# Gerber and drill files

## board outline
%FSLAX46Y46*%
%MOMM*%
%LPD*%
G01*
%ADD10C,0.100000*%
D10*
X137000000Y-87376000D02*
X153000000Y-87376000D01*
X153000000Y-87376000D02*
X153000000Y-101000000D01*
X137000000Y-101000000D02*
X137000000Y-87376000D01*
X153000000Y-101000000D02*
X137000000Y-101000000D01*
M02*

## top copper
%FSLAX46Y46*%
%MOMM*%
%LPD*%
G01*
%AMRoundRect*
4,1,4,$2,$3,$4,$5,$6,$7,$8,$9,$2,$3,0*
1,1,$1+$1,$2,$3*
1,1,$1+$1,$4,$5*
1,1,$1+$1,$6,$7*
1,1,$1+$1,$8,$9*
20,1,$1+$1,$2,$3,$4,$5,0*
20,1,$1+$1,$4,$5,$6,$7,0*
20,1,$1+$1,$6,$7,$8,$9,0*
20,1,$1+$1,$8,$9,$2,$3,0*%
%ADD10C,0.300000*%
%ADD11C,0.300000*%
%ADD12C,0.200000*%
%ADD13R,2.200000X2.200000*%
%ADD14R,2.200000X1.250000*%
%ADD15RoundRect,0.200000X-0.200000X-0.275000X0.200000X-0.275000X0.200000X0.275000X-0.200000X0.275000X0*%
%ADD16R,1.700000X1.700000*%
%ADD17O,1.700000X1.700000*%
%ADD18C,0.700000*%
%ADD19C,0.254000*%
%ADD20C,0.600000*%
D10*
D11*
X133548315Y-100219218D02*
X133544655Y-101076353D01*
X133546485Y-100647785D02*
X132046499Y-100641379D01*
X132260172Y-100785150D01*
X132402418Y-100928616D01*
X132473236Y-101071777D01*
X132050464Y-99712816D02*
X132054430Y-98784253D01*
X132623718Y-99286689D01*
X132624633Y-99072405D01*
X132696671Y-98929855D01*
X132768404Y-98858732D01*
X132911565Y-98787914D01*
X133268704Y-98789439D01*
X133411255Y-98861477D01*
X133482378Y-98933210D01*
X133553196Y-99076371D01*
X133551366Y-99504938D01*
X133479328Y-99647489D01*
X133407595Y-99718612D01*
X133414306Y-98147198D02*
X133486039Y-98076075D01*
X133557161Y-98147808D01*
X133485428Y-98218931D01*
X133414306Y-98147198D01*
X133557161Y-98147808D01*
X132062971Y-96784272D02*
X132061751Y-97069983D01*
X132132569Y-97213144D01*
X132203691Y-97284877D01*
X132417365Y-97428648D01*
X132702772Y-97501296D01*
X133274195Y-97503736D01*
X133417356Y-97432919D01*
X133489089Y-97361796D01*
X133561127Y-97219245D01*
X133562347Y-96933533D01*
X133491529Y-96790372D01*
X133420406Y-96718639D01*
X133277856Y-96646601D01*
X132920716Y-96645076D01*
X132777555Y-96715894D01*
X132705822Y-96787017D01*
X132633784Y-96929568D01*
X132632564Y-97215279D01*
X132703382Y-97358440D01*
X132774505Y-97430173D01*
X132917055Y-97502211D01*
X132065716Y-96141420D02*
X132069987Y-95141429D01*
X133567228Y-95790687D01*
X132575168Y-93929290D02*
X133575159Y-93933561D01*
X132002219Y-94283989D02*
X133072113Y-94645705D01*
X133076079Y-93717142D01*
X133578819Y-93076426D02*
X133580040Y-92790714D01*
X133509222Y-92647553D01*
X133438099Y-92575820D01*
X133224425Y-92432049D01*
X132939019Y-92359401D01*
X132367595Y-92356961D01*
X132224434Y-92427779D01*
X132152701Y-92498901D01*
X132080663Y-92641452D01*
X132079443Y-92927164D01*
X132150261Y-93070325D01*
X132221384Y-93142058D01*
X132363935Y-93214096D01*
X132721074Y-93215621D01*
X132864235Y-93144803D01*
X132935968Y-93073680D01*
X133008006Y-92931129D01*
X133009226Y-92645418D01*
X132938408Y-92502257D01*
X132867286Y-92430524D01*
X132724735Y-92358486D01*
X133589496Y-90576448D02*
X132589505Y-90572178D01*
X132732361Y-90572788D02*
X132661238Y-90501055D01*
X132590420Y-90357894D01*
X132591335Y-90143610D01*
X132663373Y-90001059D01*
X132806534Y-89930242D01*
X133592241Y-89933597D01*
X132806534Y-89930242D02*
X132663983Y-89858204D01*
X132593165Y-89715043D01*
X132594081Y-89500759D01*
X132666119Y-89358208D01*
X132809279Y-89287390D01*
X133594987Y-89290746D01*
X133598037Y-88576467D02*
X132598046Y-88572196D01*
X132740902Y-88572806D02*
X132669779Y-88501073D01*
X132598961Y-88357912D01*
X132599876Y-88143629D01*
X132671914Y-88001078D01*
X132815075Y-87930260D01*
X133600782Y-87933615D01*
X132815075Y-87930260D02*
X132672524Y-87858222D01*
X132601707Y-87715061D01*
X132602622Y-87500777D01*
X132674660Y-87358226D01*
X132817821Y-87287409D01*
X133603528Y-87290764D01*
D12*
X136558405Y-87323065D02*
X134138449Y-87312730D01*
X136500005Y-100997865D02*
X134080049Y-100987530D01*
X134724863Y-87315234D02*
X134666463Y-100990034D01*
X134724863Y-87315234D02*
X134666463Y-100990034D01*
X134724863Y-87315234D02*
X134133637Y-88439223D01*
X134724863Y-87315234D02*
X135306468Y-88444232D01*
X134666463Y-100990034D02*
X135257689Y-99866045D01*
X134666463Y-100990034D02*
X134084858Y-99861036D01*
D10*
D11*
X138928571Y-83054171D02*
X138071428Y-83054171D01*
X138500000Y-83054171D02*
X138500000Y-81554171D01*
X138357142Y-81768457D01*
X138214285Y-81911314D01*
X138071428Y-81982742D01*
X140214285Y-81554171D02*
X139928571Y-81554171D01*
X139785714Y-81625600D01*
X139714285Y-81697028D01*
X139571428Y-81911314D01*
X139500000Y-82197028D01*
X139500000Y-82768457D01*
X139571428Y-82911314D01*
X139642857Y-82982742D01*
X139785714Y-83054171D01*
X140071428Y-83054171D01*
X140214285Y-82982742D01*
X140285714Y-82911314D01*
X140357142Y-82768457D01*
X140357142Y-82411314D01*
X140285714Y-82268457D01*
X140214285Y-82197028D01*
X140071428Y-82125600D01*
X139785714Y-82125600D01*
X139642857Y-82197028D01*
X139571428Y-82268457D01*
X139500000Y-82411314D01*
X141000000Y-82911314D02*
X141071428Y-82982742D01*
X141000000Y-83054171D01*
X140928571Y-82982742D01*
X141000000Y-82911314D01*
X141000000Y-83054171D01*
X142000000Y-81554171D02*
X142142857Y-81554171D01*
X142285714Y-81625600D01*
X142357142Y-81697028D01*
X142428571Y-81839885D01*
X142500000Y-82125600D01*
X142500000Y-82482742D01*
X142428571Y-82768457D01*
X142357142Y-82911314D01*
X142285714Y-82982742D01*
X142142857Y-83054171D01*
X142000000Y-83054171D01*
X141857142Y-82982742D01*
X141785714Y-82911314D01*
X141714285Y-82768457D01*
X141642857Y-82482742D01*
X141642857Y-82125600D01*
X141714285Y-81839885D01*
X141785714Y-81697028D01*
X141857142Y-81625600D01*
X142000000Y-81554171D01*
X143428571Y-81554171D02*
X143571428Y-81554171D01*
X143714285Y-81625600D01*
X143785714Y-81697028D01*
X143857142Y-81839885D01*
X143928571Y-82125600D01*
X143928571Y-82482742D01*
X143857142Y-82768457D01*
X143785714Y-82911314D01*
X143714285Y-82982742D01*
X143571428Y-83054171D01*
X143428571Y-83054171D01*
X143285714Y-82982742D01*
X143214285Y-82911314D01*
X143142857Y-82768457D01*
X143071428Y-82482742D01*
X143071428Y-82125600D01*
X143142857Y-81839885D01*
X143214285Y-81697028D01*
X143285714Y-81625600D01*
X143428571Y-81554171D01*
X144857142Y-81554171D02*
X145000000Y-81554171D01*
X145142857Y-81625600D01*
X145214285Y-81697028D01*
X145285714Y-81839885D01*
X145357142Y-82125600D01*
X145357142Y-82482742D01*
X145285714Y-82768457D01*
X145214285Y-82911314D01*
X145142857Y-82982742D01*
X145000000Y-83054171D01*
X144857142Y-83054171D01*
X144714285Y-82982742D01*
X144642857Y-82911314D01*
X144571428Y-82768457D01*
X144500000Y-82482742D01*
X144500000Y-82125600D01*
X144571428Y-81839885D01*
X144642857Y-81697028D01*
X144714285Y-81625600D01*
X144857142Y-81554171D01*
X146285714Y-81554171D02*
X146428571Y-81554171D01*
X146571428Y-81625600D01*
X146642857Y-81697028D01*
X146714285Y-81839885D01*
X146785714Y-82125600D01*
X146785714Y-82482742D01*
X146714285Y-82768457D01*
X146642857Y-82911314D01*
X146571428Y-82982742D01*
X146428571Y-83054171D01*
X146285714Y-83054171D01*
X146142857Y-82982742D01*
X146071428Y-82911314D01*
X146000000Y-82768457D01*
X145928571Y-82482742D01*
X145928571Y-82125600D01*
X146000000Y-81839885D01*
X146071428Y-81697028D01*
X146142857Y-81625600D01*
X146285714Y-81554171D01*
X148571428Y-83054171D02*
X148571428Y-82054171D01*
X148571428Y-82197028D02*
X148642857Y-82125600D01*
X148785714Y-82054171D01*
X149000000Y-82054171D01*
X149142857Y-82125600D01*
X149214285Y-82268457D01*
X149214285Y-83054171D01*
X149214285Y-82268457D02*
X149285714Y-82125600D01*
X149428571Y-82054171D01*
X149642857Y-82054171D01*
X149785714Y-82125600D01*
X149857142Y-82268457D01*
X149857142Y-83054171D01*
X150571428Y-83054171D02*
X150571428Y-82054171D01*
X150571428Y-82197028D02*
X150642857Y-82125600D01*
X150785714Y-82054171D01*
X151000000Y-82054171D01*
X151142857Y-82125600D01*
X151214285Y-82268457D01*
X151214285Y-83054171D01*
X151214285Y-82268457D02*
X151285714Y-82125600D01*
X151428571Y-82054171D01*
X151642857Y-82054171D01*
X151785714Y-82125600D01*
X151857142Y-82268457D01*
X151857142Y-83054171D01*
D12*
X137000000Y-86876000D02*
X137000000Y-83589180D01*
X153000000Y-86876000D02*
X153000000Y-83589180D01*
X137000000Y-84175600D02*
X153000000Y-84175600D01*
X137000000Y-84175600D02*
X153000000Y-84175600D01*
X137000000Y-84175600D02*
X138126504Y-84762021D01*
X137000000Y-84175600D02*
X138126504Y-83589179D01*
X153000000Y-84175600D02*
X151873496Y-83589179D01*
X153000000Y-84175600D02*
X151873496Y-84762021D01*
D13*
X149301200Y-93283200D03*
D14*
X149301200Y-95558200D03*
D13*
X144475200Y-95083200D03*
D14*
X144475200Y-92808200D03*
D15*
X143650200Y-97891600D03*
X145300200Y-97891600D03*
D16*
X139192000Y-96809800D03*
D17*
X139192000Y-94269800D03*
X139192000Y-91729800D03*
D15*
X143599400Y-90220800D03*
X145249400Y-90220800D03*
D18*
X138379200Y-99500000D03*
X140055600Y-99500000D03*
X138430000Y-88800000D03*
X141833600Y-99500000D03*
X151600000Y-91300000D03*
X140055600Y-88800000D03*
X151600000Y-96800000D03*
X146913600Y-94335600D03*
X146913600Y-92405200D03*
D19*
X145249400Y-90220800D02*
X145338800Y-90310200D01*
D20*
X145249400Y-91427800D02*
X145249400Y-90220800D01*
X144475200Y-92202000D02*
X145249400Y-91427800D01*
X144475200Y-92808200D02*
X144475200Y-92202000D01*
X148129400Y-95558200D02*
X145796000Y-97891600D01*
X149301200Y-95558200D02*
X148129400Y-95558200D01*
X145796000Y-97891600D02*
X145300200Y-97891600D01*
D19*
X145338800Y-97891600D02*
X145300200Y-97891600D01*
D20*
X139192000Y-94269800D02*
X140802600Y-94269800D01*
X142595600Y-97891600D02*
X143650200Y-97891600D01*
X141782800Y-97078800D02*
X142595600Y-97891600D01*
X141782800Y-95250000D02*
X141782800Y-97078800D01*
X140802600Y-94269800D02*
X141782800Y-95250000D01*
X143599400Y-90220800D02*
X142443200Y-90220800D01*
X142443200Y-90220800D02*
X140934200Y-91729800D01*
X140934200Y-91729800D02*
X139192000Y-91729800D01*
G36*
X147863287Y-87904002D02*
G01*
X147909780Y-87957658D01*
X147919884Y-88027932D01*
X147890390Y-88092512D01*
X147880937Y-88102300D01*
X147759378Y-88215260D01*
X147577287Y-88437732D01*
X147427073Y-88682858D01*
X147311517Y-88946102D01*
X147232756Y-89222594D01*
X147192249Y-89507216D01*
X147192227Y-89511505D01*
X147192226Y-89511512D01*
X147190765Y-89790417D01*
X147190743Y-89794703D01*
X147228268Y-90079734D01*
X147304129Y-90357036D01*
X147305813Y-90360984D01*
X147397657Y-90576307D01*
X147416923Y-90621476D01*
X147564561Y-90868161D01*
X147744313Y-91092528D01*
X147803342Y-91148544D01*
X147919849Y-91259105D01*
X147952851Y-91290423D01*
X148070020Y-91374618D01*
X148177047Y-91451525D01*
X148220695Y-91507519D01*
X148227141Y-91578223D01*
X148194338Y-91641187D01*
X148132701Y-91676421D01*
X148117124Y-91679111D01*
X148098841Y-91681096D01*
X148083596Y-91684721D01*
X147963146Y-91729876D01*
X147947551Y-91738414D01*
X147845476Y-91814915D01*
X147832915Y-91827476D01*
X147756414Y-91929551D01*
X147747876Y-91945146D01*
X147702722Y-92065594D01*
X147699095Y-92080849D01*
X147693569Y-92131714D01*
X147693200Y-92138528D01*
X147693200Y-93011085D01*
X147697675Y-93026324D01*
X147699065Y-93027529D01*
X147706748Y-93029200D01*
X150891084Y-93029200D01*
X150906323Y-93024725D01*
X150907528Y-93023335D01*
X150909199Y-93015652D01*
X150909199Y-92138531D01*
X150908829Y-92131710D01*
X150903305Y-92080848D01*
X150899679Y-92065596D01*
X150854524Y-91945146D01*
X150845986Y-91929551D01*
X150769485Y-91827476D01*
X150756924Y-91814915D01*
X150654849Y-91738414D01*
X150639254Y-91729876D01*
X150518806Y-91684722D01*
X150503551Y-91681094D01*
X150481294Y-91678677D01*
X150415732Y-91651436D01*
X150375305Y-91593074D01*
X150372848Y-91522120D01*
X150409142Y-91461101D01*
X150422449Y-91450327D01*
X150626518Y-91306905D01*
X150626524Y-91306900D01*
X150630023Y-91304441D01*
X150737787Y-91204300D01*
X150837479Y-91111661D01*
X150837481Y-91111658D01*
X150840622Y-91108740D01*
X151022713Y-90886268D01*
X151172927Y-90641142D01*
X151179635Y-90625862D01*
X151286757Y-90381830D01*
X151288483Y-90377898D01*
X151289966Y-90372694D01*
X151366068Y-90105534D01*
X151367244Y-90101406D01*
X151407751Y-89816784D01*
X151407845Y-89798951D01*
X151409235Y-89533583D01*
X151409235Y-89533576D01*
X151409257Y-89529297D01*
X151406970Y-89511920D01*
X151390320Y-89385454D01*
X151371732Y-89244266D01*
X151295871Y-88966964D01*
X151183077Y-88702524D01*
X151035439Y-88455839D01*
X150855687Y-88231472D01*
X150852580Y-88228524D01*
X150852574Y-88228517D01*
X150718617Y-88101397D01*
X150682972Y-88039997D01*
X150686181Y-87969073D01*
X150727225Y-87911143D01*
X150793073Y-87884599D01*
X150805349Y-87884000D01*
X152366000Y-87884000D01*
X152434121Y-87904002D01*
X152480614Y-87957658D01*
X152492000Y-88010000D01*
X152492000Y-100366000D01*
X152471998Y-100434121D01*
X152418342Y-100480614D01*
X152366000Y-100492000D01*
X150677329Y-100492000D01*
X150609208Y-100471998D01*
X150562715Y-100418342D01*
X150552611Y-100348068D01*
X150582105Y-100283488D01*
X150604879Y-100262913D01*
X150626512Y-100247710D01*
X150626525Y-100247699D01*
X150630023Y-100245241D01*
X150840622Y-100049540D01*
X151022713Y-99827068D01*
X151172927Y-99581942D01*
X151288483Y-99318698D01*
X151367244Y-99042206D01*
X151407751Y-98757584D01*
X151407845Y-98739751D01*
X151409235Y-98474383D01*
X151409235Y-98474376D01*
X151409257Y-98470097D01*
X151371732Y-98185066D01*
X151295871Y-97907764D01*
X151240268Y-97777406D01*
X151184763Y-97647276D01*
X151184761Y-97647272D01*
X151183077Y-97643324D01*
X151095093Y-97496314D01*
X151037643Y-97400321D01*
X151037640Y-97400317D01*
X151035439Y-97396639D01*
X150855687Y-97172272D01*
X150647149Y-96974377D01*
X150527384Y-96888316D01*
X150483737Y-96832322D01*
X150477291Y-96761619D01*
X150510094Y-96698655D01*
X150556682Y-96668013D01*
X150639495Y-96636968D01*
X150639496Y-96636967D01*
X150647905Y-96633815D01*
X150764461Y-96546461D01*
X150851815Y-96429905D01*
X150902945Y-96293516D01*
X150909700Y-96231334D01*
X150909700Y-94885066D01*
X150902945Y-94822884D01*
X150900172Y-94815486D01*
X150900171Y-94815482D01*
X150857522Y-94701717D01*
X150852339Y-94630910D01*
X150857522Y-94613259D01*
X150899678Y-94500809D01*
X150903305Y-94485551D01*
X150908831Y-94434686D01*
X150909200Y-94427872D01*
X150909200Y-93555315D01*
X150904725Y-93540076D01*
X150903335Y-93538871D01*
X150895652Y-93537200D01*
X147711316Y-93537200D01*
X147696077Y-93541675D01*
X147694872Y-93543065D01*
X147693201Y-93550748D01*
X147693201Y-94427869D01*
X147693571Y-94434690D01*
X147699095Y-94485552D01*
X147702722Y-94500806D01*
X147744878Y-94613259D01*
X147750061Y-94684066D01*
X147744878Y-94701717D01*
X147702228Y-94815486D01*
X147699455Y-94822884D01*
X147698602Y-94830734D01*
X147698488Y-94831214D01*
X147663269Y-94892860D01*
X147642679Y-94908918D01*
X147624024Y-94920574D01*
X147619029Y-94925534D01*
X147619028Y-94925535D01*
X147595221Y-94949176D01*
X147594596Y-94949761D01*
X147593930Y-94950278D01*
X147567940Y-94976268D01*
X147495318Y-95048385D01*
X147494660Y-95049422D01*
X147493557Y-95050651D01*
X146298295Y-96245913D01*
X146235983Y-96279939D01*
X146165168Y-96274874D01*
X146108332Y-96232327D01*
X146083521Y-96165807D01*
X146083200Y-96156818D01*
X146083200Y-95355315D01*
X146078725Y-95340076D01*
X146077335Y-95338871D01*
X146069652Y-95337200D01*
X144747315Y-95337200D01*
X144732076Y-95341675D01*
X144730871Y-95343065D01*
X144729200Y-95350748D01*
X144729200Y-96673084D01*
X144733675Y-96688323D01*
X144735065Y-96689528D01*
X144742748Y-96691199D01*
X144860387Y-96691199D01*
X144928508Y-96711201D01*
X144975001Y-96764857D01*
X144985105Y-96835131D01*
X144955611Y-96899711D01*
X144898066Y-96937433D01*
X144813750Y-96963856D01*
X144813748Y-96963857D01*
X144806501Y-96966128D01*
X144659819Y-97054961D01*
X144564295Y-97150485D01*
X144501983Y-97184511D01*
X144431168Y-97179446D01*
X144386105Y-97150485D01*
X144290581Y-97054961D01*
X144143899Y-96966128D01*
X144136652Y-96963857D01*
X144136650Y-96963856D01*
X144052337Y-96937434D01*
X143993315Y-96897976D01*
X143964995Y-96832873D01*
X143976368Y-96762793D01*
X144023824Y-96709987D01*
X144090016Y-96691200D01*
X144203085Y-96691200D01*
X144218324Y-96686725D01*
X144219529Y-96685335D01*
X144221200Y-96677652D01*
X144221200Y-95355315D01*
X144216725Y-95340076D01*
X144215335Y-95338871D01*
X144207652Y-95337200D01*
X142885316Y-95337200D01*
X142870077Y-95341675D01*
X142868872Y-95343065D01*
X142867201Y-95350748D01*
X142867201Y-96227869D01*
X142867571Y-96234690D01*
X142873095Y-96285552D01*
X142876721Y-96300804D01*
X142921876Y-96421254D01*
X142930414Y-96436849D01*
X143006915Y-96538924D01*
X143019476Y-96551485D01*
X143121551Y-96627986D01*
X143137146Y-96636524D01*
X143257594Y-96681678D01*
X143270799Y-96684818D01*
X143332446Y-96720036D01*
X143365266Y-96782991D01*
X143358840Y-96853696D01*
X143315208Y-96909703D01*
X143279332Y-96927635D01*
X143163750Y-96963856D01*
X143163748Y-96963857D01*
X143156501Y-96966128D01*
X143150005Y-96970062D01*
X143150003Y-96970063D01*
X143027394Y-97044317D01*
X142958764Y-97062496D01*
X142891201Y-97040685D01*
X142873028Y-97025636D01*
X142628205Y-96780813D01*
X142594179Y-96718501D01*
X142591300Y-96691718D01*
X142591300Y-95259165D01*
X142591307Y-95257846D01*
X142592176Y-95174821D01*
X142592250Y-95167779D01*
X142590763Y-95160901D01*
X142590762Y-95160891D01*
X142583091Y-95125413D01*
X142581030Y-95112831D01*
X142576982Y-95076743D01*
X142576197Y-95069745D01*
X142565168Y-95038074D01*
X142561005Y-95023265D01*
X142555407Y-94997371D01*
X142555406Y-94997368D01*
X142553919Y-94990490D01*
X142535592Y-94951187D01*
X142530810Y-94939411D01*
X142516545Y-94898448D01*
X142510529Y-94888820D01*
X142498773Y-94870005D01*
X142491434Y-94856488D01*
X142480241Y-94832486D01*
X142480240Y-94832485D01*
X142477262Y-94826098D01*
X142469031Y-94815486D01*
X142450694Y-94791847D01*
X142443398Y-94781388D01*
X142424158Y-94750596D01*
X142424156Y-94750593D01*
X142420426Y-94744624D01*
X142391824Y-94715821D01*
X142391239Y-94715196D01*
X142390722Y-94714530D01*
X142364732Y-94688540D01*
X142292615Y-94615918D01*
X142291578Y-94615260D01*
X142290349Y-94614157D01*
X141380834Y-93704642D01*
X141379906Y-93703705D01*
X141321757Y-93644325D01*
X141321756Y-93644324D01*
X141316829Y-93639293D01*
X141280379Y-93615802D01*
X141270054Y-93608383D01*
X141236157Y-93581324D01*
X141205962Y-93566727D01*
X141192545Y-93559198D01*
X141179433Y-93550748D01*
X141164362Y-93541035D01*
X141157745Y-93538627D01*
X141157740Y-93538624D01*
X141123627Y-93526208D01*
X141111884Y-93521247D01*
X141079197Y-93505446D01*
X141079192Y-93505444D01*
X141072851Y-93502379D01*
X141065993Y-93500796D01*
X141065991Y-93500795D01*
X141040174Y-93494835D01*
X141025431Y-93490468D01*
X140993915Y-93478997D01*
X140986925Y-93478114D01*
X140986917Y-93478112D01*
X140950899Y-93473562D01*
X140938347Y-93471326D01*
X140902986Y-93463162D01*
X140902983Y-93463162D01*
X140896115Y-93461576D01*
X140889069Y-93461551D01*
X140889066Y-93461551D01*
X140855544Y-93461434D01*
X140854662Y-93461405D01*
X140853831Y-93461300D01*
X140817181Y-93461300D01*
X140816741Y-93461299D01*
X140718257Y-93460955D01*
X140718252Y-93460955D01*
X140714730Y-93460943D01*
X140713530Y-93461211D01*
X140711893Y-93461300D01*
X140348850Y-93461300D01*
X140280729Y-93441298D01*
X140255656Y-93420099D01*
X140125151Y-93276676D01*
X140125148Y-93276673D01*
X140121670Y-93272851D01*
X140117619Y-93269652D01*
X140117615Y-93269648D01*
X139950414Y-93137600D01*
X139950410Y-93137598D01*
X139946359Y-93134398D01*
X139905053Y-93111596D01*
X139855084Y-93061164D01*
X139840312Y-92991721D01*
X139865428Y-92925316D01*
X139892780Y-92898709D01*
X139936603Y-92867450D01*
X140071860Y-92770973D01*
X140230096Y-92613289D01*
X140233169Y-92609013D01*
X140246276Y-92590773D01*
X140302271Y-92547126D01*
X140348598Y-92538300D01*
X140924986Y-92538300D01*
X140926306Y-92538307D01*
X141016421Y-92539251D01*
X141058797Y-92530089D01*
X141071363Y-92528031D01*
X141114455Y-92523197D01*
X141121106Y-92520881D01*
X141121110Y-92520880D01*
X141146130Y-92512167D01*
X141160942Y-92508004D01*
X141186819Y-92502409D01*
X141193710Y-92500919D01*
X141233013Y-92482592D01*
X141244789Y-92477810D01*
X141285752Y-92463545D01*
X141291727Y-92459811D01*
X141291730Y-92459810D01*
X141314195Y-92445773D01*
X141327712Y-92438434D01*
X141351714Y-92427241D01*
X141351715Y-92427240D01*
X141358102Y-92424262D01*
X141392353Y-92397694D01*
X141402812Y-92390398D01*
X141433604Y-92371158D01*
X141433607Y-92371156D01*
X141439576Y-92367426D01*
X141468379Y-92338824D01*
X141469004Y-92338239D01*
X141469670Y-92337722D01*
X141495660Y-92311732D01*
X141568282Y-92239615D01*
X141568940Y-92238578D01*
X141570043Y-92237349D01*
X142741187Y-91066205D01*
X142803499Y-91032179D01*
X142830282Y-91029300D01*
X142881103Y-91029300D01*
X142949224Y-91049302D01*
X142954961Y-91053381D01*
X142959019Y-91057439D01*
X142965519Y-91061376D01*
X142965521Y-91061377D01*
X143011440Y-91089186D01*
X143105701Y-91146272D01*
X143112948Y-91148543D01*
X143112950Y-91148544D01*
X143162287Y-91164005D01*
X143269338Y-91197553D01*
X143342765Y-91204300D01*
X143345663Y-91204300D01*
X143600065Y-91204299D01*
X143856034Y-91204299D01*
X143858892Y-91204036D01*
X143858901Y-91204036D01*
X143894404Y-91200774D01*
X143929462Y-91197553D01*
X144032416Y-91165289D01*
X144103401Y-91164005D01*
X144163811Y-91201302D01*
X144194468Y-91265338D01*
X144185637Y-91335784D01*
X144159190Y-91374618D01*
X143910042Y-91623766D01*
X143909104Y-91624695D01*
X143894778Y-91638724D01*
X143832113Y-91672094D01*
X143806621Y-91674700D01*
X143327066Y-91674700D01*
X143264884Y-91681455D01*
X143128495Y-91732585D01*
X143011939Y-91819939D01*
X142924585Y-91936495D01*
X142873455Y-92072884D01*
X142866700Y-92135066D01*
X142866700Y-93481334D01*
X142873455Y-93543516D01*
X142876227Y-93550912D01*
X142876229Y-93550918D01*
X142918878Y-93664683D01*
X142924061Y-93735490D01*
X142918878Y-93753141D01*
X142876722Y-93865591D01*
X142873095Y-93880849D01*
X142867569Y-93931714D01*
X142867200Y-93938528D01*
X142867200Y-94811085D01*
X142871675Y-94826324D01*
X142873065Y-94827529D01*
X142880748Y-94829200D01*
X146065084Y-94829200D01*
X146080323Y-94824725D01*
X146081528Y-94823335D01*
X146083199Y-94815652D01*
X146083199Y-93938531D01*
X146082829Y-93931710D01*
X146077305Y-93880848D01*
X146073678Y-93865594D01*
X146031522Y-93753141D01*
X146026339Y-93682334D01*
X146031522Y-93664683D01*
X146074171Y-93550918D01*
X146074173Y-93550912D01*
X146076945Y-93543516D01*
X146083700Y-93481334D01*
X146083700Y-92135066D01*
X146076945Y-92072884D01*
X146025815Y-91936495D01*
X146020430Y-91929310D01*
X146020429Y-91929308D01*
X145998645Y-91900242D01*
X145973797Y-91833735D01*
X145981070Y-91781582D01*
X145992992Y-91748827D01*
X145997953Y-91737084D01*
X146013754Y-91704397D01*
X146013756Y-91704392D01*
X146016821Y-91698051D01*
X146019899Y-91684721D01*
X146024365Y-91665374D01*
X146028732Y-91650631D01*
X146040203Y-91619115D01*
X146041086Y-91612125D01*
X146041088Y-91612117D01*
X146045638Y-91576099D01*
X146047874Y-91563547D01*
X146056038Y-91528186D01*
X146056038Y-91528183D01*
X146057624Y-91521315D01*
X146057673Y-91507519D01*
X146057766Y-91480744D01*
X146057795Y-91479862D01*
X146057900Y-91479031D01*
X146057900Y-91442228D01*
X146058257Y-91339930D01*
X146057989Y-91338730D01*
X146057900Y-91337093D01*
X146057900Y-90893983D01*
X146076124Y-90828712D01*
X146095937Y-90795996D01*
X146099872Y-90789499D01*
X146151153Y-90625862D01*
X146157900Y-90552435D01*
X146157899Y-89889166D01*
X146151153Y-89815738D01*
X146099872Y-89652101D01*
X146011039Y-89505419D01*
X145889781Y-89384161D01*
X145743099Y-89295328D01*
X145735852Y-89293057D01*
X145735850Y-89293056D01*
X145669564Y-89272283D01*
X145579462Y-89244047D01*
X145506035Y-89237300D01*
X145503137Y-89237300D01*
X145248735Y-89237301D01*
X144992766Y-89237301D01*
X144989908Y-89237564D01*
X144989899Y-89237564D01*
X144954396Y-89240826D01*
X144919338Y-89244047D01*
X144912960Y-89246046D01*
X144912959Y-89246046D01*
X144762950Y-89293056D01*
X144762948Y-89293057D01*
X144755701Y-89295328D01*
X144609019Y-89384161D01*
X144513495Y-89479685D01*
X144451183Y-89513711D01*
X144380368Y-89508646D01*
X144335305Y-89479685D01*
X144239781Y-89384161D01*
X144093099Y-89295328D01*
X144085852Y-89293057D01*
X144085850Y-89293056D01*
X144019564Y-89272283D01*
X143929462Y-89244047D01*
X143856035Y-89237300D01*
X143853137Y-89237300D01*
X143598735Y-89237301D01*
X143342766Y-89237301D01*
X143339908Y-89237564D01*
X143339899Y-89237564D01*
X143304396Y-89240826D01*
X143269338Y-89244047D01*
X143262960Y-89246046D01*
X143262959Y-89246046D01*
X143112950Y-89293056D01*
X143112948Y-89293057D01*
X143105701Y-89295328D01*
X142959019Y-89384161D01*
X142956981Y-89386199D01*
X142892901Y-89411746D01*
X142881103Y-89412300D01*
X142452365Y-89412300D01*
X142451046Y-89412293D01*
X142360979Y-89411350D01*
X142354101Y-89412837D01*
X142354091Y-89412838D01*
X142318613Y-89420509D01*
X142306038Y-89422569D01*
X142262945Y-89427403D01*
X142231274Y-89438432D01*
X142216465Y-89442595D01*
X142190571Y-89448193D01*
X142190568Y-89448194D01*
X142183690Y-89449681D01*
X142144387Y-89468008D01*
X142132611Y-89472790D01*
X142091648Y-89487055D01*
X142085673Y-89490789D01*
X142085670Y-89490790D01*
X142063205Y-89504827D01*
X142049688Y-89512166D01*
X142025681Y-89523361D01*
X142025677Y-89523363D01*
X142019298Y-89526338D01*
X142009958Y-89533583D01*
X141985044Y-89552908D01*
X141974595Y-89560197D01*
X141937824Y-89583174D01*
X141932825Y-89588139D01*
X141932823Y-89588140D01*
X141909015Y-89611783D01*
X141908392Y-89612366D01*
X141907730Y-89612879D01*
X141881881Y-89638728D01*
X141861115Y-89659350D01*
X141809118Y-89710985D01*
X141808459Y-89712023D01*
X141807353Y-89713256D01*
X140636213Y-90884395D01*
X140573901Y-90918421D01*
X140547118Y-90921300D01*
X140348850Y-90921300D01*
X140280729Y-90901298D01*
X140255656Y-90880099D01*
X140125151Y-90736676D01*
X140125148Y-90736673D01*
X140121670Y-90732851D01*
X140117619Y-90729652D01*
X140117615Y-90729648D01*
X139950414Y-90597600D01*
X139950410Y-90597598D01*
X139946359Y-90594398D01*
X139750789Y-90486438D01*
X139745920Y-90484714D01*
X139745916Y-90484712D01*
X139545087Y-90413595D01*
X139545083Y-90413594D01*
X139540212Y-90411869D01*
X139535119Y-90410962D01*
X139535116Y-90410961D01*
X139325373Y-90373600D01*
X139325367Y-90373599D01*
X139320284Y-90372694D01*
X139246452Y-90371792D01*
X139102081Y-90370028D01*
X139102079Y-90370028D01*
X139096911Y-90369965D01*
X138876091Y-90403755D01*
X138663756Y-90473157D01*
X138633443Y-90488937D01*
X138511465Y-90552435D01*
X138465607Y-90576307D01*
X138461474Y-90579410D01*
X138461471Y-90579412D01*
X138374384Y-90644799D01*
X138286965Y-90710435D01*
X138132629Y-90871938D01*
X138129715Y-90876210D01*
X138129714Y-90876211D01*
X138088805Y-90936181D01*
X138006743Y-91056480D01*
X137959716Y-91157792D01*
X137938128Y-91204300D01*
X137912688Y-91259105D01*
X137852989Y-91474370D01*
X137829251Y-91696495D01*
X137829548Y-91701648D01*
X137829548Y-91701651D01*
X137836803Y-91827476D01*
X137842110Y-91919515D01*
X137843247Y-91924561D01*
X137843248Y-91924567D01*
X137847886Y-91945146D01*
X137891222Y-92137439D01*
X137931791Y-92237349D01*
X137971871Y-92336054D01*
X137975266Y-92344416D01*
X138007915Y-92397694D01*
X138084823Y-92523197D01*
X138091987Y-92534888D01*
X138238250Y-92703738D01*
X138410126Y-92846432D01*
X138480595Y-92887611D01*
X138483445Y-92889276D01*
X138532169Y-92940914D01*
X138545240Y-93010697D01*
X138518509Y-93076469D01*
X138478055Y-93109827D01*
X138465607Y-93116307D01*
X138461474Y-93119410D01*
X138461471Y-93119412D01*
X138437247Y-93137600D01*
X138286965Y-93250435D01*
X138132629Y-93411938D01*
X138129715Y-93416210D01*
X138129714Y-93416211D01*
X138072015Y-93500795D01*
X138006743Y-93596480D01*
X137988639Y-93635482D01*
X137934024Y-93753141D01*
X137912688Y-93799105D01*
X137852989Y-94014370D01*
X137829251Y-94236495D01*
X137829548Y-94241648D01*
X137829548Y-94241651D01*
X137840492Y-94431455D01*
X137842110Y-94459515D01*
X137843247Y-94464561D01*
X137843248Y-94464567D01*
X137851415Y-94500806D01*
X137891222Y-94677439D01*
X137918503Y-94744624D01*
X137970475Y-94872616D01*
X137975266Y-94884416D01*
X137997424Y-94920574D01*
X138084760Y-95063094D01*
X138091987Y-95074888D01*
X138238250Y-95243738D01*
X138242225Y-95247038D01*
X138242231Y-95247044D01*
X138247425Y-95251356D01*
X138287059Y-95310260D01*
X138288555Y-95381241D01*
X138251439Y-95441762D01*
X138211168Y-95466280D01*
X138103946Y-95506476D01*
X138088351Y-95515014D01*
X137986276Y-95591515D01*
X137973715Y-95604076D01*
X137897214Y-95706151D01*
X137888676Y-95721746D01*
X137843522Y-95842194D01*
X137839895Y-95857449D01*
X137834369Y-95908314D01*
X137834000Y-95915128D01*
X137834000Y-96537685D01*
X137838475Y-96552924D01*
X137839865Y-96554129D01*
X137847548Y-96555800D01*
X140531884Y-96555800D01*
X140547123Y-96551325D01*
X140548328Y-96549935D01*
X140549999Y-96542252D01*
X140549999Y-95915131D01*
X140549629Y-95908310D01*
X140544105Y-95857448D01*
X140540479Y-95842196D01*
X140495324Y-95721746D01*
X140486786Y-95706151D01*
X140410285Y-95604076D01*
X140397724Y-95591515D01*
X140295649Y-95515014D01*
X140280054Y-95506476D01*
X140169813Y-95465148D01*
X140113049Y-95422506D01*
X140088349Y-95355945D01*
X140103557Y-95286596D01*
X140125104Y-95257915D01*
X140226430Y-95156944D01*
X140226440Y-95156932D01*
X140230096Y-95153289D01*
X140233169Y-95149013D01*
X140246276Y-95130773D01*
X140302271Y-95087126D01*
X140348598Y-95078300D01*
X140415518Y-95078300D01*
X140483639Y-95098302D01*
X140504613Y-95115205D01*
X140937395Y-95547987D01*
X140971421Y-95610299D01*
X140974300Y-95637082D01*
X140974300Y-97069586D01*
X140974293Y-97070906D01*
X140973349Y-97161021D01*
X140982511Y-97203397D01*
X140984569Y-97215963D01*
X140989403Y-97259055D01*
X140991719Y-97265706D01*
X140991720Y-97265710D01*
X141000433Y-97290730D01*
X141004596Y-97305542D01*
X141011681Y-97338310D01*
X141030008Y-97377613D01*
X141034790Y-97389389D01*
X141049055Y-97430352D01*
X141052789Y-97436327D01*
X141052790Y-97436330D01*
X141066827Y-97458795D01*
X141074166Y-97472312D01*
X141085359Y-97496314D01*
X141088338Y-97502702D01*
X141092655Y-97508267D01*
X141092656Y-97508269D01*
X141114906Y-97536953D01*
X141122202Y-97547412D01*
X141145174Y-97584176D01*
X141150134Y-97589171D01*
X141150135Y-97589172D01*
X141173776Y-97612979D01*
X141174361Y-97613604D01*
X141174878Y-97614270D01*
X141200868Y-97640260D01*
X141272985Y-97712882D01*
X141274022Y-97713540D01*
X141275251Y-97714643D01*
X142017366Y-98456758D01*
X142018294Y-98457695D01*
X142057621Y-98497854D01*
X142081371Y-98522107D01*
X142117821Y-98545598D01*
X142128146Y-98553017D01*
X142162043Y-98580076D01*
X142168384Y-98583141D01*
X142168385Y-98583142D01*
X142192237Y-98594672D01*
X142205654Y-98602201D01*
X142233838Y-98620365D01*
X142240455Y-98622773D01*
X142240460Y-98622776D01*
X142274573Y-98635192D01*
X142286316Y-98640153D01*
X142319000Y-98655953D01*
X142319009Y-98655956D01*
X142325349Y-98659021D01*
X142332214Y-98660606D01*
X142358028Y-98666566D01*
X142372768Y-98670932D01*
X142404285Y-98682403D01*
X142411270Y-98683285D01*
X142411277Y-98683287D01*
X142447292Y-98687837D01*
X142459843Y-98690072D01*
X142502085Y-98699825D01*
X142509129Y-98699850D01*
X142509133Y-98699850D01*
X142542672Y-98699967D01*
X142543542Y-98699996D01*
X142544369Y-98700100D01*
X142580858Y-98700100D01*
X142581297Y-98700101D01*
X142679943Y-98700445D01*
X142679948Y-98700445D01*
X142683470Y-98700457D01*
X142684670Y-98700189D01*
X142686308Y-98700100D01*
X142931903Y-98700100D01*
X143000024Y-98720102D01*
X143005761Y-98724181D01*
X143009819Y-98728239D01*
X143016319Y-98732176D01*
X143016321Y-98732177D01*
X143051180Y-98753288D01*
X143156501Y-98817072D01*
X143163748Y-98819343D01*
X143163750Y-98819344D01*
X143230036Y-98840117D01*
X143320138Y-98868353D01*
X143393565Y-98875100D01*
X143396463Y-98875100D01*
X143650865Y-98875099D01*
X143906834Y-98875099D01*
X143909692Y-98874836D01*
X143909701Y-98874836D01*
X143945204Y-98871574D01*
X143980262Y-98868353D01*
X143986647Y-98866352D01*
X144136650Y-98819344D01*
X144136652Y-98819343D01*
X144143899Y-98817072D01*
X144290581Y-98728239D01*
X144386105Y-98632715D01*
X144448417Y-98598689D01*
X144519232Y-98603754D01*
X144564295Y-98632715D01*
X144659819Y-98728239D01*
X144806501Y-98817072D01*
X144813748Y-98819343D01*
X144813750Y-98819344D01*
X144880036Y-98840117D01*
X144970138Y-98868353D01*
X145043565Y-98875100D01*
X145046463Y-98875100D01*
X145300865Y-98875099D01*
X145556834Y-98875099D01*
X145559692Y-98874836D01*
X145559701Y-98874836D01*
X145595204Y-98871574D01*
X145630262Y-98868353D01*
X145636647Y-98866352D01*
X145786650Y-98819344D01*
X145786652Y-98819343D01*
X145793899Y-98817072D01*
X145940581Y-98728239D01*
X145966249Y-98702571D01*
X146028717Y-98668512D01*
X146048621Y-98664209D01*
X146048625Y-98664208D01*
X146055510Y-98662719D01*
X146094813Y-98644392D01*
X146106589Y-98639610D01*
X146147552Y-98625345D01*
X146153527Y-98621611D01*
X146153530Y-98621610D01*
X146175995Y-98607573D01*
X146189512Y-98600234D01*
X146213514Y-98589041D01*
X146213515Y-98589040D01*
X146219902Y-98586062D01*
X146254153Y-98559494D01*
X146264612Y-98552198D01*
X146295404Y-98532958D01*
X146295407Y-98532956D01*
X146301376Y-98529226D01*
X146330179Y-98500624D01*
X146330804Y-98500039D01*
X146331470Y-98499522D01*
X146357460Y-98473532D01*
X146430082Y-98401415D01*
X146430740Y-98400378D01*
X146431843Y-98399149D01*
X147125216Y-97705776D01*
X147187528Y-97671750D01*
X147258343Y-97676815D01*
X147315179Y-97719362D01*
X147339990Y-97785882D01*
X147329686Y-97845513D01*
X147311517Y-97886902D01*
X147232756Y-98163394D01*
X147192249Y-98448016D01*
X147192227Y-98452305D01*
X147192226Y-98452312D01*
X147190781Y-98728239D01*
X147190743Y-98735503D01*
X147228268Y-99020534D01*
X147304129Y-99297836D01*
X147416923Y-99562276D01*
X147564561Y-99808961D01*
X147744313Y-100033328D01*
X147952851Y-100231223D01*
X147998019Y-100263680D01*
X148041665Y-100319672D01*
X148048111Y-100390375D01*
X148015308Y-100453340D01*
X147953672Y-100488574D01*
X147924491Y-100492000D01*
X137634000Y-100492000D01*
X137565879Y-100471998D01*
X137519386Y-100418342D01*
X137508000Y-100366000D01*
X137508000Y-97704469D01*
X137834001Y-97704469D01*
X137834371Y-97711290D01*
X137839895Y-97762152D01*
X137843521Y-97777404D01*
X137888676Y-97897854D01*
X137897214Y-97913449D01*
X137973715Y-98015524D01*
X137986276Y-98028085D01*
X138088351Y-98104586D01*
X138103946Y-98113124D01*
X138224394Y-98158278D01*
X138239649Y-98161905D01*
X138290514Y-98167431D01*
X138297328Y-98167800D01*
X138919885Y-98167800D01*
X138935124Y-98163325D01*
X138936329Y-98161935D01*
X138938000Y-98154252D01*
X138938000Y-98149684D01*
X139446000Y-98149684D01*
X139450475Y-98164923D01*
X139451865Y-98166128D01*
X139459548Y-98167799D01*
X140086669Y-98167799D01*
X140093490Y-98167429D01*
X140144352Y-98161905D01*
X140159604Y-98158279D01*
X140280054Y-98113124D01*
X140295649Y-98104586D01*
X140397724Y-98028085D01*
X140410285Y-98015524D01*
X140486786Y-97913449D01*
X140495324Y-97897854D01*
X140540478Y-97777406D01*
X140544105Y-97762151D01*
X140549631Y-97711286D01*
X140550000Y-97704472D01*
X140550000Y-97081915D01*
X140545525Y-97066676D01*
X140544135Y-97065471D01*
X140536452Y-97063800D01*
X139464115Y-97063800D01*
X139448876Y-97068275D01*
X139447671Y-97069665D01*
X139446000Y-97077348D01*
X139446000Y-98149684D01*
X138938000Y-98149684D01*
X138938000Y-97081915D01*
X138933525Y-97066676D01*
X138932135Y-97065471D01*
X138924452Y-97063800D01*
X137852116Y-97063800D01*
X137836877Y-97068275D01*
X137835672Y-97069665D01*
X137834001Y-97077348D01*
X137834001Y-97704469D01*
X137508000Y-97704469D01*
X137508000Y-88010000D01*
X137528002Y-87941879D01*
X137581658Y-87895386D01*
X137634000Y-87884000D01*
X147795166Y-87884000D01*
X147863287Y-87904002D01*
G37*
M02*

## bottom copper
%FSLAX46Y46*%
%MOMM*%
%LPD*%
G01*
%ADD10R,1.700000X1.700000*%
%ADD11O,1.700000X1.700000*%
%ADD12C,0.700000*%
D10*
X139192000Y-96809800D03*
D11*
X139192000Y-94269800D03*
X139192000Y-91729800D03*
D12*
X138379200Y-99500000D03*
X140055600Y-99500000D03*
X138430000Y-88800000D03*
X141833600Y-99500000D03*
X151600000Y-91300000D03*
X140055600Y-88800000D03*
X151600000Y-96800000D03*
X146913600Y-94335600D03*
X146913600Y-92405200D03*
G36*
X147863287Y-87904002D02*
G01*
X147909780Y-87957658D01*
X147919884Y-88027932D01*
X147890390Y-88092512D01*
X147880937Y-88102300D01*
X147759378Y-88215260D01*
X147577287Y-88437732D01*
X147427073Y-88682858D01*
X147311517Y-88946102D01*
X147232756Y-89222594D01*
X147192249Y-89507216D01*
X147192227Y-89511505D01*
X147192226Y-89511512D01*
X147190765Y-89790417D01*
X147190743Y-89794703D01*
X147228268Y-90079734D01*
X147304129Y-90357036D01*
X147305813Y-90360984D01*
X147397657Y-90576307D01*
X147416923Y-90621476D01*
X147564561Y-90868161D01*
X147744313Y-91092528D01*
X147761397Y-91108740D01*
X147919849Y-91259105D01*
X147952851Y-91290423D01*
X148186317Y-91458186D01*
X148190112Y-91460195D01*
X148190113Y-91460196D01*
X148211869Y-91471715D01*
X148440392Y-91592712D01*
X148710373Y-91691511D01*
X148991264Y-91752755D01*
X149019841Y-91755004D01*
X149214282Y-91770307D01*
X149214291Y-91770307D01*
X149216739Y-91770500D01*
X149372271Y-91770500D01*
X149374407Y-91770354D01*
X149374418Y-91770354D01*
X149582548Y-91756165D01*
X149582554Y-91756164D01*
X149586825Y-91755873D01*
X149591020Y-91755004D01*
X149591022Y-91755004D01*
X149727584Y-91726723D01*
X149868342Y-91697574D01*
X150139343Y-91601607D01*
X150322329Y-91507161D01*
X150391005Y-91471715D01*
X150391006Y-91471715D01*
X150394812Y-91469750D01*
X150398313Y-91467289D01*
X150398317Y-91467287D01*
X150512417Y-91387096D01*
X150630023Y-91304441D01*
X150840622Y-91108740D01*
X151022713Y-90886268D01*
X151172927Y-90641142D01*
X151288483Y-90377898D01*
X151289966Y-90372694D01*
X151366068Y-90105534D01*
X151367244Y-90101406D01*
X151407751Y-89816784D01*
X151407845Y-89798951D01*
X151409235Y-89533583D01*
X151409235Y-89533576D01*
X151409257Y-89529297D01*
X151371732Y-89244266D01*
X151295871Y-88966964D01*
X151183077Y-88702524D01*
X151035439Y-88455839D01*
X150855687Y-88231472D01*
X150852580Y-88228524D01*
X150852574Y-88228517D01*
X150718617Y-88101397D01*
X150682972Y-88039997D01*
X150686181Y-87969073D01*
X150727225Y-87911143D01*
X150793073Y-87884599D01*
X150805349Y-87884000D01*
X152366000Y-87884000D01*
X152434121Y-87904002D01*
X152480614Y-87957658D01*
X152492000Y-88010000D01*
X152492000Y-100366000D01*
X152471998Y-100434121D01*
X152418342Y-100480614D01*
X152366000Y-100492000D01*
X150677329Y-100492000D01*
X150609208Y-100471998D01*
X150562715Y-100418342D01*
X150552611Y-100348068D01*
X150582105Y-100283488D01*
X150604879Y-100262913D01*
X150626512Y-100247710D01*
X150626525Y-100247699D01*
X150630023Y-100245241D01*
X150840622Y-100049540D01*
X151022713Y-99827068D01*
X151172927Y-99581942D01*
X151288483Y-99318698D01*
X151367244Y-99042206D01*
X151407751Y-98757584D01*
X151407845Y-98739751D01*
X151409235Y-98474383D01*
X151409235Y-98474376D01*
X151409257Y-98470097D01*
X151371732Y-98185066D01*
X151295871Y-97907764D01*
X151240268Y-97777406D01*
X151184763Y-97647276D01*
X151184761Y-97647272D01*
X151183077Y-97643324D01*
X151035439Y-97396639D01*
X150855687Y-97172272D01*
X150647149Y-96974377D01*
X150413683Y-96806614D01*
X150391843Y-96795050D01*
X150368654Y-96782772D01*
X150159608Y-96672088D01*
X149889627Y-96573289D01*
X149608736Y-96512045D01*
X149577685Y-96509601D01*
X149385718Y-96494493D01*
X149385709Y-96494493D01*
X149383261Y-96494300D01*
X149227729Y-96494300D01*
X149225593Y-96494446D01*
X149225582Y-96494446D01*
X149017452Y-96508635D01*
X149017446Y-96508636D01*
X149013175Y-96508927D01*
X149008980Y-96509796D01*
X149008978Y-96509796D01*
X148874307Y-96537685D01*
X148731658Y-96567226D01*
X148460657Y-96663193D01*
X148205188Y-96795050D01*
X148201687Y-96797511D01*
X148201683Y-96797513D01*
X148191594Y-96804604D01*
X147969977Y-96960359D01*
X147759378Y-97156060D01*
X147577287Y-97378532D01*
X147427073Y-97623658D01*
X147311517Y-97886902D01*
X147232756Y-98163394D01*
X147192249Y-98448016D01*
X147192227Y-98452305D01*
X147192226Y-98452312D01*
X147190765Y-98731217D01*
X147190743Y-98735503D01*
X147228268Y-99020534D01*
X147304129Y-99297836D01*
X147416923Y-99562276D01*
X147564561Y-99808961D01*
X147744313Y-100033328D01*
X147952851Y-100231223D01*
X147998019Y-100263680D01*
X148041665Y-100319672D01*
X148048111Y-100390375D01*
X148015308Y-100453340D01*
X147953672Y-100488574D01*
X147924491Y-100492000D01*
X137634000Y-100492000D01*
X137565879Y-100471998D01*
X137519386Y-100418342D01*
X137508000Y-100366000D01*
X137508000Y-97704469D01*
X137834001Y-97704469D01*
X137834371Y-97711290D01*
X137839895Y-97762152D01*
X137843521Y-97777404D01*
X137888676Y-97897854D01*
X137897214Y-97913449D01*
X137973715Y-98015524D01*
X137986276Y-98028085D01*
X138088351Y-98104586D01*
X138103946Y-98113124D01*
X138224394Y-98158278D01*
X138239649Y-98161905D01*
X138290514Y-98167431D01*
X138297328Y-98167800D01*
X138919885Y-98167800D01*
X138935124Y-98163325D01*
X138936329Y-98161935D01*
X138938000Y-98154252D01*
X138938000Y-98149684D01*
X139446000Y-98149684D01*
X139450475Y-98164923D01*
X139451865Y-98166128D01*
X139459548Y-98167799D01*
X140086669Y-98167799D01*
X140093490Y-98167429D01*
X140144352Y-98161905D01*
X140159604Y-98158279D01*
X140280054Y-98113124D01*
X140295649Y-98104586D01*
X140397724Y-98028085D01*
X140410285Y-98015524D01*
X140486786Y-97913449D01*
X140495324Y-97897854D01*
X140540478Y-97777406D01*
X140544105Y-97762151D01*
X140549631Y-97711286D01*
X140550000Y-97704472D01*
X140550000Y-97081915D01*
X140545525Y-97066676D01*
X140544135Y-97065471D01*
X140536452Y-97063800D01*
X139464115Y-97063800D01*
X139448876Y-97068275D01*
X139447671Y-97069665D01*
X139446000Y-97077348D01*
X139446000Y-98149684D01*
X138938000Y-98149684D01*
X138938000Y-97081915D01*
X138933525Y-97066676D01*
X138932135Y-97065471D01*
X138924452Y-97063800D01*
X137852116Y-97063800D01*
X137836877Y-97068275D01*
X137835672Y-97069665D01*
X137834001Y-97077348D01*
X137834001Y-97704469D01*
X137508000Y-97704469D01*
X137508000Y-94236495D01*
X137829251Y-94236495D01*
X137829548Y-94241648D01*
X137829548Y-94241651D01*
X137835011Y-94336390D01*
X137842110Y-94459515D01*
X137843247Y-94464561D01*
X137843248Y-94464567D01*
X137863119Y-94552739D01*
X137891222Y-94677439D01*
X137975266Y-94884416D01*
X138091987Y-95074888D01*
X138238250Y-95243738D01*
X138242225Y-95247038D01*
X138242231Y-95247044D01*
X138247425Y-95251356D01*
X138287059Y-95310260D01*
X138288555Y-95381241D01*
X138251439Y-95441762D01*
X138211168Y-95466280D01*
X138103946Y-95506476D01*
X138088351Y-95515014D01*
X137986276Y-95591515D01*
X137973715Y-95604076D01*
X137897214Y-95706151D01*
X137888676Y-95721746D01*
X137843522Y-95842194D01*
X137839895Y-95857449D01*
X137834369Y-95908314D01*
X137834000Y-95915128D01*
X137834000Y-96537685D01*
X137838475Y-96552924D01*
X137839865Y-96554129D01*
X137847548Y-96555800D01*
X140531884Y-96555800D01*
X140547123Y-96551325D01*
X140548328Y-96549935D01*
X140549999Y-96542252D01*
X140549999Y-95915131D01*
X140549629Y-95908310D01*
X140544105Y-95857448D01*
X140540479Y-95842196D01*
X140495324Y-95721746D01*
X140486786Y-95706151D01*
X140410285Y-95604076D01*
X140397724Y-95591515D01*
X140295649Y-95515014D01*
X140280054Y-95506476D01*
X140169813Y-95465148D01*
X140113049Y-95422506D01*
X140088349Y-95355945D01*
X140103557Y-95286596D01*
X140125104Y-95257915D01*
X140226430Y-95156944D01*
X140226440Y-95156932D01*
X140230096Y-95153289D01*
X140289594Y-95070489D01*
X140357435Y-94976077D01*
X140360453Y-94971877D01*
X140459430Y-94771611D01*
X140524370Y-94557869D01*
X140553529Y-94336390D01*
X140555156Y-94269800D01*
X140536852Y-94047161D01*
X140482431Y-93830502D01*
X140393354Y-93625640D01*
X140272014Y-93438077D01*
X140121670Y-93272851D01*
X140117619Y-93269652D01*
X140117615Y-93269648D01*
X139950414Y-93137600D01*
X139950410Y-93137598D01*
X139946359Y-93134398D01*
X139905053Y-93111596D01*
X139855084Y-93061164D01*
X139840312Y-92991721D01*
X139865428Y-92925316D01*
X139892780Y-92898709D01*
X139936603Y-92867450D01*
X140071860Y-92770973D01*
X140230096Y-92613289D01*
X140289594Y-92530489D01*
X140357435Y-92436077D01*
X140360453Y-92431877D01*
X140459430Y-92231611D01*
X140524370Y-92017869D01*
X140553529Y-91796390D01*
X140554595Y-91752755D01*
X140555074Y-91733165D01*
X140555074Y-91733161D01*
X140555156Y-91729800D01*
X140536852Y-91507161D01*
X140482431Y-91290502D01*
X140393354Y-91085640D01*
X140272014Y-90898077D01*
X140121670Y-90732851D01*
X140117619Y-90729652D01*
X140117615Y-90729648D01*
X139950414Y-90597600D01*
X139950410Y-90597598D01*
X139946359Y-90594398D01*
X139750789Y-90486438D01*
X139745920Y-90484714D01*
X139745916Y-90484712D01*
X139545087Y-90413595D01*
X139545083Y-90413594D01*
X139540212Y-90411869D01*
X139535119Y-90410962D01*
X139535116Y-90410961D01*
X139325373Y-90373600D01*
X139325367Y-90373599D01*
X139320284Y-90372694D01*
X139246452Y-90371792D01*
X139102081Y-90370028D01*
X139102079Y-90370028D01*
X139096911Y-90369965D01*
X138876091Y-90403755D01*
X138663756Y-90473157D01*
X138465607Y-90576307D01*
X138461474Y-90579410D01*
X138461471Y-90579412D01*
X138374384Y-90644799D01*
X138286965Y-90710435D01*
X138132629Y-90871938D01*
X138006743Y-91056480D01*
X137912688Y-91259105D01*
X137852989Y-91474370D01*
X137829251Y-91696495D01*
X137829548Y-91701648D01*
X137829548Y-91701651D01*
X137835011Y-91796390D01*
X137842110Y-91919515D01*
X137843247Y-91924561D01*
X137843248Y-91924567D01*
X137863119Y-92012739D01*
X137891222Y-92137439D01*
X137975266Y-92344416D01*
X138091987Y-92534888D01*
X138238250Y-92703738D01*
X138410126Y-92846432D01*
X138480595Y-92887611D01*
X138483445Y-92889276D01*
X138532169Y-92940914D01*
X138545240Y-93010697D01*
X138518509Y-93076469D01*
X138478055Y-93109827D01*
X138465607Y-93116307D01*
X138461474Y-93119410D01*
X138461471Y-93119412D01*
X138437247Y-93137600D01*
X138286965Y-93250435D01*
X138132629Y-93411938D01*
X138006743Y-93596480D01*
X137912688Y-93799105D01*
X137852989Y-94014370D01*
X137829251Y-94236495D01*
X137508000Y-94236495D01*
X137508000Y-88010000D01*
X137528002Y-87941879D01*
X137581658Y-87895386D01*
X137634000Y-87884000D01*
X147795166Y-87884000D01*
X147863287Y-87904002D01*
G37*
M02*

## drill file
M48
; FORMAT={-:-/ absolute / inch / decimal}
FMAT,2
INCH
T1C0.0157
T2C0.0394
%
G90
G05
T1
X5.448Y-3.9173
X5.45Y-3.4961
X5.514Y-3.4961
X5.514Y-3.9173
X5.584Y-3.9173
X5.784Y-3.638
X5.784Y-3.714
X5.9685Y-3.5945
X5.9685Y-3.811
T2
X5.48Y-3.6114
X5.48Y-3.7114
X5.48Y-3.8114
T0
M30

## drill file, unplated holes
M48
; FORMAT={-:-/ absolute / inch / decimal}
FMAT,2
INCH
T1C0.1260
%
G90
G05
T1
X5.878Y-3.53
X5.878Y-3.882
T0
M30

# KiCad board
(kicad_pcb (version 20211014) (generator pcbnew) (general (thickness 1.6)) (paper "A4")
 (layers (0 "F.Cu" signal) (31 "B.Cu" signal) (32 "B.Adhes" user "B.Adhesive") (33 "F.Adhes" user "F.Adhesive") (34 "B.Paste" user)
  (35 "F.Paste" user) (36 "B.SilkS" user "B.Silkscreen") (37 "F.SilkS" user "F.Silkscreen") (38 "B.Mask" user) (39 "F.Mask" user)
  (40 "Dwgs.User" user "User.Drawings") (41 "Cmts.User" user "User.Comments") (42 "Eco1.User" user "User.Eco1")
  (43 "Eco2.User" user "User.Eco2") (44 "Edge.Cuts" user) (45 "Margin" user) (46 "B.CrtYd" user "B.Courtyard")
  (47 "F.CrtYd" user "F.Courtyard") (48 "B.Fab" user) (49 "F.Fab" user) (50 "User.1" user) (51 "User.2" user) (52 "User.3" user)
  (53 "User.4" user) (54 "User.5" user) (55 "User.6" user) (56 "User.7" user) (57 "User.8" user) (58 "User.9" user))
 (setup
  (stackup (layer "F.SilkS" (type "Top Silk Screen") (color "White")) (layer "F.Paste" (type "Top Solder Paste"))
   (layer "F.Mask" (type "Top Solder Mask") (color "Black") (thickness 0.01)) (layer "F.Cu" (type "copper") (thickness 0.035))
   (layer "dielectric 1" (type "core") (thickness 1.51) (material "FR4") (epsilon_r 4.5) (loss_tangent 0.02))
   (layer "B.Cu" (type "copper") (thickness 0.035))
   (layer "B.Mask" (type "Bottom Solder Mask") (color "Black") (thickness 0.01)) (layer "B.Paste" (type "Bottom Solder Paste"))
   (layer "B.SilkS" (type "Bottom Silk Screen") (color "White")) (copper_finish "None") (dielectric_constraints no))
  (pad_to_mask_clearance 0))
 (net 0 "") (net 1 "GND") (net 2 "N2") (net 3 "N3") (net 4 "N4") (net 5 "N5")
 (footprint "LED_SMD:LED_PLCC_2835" (layer "F.Cu") (at 149.3012 94.1832 -90)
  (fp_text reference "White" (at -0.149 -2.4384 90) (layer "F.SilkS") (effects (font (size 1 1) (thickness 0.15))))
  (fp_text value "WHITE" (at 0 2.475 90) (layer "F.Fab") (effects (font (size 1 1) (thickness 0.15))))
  (pad "1" smd rect (at -0.9 0 270) (size 2.2 2.2) (layers "F.Cu" "F.Paste" "F.Mask") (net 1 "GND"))
  (pad "2" smd rect (at 1.375 0 270) (size 1.25 2.2) (layers "F.Cu" "F.Paste" "F.Mask") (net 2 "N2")))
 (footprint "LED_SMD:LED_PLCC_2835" (layer "F.Cu") (at 144.4752 94.1832 90)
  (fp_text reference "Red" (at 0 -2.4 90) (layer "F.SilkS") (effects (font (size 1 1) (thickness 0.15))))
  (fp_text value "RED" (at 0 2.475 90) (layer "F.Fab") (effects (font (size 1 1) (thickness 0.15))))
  (pad "1" smd rect (at -0.9 0 90) (size 2.2 2.2) (layers "F.Cu" "F.Paste" "F.Mask") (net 1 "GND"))
  (pad "2" smd rect (at 1.375 0 90) (size 1.25 2.2) (layers "F.Cu" "F.Paste" "F.Mask") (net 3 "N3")))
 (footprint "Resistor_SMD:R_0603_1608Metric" (layer "F.Cu") (at 144.4752 97.8916)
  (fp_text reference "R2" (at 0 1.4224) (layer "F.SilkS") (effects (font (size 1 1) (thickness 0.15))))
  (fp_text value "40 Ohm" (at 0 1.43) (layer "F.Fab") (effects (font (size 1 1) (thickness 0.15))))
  (pad "1" smd roundrect (at -0.825 0) (size 0.8 0.95) (layers "F.Cu" "F.Paste" "F.Mask") (roundrect_rratio 0.25) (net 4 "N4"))
  (pad "2" smd roundrect (at 0.825 0) (size 0.8 0.95) (layers "F.Cu" "F.Paste" "F.Mask") (roundrect_rratio 0.25) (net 2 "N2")))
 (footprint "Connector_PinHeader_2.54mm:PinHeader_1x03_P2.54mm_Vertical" (layer "F.Cu") (at 139.192 96.8098 180)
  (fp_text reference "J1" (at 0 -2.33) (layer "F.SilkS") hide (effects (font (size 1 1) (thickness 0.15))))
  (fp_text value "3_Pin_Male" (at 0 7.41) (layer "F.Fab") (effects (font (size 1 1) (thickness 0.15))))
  (pad "1" thru_hole rect (at 0 0 180) (size 1.7 1.7) (drill 1) (layers *.Cu *.Mask) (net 1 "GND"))
  (pad "2" thru_hole oval (at 0 2.54 180) (size 1.7 1.7) (drill 1) (layers *.Cu *.Mask) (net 4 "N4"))
  (pad "3" thru_hole oval (at 0 5.08 180) (size 1.7 1.7) (drill 1) (layers *.Cu *.Mask) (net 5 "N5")))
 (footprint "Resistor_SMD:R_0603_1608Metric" (layer "F.Cu") (at 144.4244 90.2208)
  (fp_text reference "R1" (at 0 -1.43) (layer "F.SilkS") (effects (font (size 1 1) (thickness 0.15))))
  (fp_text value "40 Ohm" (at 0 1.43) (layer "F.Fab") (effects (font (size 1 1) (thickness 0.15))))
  (pad "1" smd roundrect (at -0.825 0) (size 0.8 0.95) (layers "F.Cu" "F.Paste" "F.Mask") (roundrect_rratio 0.25) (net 5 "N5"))
  (pad "2" smd roundrect (at 0.825 0) (size 0.8 0.95) (layers "F.Cu" "F.Paste" "F.Mask") (roundrect_rratio 0.25) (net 3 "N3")))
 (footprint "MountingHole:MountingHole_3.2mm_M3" (layer "F.Cu") (at 149.3 98.6028)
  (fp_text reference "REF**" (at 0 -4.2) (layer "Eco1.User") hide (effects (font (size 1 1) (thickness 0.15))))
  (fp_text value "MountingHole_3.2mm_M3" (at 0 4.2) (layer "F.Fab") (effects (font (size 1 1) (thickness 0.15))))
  (pad "" np_thru_hole circle (at 0 0) (size 3.2 3.2) (drill 3.2) (layers *.Cu *.Mask)))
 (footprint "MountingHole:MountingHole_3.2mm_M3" (layer "F.Cu") (at 149.3 89.662)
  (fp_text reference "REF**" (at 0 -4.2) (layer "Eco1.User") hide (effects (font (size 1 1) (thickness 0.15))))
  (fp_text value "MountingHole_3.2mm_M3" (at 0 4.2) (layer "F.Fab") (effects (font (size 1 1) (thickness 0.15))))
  (pad "" np_thru_hole circle (at 0 0) (size 3.2 3.2) (drill 3.2) (layers *.Cu *.Mask)))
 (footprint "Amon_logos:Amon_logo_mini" (layer "B.Cu") (at 144.526 94.4372 90)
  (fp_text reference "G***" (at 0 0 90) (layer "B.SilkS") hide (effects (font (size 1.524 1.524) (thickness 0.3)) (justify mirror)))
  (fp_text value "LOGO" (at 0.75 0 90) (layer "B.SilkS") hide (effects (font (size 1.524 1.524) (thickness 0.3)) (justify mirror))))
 (gr_line (start 137 87.376) (end 153 87.376) (layer "Edge.Cuts") (width 0.1))
 (gr_line (start 153 87.376) (end 153 101) (layer "Edge.Cuts") (width 0.1))
 (gr_line (start 137 101) (end 137 87.376) (layer "Edge.Cuts") (width 0.1))
 (gr_line (start 153 101) (end 137 101) (layer "Edge.Cuts") (width 0.1))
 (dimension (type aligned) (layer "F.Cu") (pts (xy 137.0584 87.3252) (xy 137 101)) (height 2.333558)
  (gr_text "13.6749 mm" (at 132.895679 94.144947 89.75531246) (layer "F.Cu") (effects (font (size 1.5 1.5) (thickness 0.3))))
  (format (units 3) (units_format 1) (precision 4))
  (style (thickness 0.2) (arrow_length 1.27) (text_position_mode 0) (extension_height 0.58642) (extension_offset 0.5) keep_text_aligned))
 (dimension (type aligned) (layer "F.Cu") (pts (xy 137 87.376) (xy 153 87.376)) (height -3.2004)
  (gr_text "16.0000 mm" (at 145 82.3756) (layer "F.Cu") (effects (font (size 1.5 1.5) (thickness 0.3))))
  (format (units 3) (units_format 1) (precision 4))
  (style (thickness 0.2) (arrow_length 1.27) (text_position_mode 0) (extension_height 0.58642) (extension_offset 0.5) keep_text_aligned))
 (segment (start 145.2494 90.2208) (end 145.3388 90.3102) (width 0.254) (layer "F.Cu") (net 3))
 (segment (start 145.2494 91.4278) (end 145.2494 90.2208) (width 0.6) (layer "F.Cu") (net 3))
 (segment (start 144.4752 92.202) (end 145.2494 91.4278) (width 0.6) (layer "F.Cu") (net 3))
 (segment (start 144.4752 92.8082) (end 144.4752 92.202) (width 0.6) (layer "F.Cu") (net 3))
 (segment (start 148.1294 95.5582) (end 145.796 97.8916) (width 0.6) (layer "F.Cu") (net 2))
 (segment (start 149.3012 95.5582) (end 148.1294 95.5582) (width 0.6) (layer "F.Cu") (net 2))
 (segment (start 145.796 97.8916) (end 145.3002 97.8916) (width 0.6) (layer "F.Cu") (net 2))
 (segment (start 145.3388 97.8916) (end 145.3002 97.8916) (width 0.254) (layer "F.Cu") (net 2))
 (segment (start 139.192 94.2698) (end 140.8026 94.2698) (width 0.6) (layer "F.Cu") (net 4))
 (segment (start 142.5956 97.8916) (end 143.6502 97.8916) (width 0.6) (layer "F.Cu") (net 4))
 (segment (start 141.7828 97.0788) (end 142.5956 97.8916) (width 0.6) (layer "F.Cu") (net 4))
 (segment (start 141.7828 95.25) (end 141.7828 97.0788) (width 0.6) (layer "F.Cu") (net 4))
 (segment (start 140.8026 94.2698) (end 141.7828 95.25) (width 0.6) (layer "F.Cu") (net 4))
 (segment (start 143.5994 90.2208) (end 142.4432 90.2208) (width 0.6) (layer "F.Cu") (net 5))
 (segment (start 142.4432 90.2208) (end 140.9342 91.7298) (width 0.6) (layer "F.Cu") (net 5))
 (segment (start 140.9342 91.7298) (end 139.192 91.7298) (width 0.6) (layer "F.Cu") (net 5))
 (via (at 138.3792 99.5) (size 0.7) (drill 0.4) (layers "F.Cu" "B.Cu") (free) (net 1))
 (via (at 140.0556 99.5) (size 0.7) (drill 0.4) (layers "F.Cu" "B.Cu") (free) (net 1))
 (via (at 138.43 88.8) (size 0.7) (drill 0.4) (layers "F.Cu" "B.Cu") (free) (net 1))
 (via (at 141.8336 99.5) (size 0.7) (drill 0.4) (layers "F.Cu" "B.Cu") (free) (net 1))
 (via (at 151.6 91.3) (size 0.7) (drill 0.4) (layers "F.Cu" "B.Cu") (free) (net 1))
 (via (at 140.0556 88.8) (size 0.7) (drill 0.4) (layers "F.Cu" "B.Cu") (free) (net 1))
 (via (at 151.6 96.8) (size 0.7) (drill 0.4) (layers "F.Cu" "B.Cu") (free) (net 1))
 (via (at 146.9136 94.3356) (size 0.7) (drill 0.4) (layers "F.Cu" "B.Cu") (free) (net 1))
 (via (at 146.9136 92.4052) (size 0.7) (drill 0.4) (layers "F.Cu" "B.Cu") (free) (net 1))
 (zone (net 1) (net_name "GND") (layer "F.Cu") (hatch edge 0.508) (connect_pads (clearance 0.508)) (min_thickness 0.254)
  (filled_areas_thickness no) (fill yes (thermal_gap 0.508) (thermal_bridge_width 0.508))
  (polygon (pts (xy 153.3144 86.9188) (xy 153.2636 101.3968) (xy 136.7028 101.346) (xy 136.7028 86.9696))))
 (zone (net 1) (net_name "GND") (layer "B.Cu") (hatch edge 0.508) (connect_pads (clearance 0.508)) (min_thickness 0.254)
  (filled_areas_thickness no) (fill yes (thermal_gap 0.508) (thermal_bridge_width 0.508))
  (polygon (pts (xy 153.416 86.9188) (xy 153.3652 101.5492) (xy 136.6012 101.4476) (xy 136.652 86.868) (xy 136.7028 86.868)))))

